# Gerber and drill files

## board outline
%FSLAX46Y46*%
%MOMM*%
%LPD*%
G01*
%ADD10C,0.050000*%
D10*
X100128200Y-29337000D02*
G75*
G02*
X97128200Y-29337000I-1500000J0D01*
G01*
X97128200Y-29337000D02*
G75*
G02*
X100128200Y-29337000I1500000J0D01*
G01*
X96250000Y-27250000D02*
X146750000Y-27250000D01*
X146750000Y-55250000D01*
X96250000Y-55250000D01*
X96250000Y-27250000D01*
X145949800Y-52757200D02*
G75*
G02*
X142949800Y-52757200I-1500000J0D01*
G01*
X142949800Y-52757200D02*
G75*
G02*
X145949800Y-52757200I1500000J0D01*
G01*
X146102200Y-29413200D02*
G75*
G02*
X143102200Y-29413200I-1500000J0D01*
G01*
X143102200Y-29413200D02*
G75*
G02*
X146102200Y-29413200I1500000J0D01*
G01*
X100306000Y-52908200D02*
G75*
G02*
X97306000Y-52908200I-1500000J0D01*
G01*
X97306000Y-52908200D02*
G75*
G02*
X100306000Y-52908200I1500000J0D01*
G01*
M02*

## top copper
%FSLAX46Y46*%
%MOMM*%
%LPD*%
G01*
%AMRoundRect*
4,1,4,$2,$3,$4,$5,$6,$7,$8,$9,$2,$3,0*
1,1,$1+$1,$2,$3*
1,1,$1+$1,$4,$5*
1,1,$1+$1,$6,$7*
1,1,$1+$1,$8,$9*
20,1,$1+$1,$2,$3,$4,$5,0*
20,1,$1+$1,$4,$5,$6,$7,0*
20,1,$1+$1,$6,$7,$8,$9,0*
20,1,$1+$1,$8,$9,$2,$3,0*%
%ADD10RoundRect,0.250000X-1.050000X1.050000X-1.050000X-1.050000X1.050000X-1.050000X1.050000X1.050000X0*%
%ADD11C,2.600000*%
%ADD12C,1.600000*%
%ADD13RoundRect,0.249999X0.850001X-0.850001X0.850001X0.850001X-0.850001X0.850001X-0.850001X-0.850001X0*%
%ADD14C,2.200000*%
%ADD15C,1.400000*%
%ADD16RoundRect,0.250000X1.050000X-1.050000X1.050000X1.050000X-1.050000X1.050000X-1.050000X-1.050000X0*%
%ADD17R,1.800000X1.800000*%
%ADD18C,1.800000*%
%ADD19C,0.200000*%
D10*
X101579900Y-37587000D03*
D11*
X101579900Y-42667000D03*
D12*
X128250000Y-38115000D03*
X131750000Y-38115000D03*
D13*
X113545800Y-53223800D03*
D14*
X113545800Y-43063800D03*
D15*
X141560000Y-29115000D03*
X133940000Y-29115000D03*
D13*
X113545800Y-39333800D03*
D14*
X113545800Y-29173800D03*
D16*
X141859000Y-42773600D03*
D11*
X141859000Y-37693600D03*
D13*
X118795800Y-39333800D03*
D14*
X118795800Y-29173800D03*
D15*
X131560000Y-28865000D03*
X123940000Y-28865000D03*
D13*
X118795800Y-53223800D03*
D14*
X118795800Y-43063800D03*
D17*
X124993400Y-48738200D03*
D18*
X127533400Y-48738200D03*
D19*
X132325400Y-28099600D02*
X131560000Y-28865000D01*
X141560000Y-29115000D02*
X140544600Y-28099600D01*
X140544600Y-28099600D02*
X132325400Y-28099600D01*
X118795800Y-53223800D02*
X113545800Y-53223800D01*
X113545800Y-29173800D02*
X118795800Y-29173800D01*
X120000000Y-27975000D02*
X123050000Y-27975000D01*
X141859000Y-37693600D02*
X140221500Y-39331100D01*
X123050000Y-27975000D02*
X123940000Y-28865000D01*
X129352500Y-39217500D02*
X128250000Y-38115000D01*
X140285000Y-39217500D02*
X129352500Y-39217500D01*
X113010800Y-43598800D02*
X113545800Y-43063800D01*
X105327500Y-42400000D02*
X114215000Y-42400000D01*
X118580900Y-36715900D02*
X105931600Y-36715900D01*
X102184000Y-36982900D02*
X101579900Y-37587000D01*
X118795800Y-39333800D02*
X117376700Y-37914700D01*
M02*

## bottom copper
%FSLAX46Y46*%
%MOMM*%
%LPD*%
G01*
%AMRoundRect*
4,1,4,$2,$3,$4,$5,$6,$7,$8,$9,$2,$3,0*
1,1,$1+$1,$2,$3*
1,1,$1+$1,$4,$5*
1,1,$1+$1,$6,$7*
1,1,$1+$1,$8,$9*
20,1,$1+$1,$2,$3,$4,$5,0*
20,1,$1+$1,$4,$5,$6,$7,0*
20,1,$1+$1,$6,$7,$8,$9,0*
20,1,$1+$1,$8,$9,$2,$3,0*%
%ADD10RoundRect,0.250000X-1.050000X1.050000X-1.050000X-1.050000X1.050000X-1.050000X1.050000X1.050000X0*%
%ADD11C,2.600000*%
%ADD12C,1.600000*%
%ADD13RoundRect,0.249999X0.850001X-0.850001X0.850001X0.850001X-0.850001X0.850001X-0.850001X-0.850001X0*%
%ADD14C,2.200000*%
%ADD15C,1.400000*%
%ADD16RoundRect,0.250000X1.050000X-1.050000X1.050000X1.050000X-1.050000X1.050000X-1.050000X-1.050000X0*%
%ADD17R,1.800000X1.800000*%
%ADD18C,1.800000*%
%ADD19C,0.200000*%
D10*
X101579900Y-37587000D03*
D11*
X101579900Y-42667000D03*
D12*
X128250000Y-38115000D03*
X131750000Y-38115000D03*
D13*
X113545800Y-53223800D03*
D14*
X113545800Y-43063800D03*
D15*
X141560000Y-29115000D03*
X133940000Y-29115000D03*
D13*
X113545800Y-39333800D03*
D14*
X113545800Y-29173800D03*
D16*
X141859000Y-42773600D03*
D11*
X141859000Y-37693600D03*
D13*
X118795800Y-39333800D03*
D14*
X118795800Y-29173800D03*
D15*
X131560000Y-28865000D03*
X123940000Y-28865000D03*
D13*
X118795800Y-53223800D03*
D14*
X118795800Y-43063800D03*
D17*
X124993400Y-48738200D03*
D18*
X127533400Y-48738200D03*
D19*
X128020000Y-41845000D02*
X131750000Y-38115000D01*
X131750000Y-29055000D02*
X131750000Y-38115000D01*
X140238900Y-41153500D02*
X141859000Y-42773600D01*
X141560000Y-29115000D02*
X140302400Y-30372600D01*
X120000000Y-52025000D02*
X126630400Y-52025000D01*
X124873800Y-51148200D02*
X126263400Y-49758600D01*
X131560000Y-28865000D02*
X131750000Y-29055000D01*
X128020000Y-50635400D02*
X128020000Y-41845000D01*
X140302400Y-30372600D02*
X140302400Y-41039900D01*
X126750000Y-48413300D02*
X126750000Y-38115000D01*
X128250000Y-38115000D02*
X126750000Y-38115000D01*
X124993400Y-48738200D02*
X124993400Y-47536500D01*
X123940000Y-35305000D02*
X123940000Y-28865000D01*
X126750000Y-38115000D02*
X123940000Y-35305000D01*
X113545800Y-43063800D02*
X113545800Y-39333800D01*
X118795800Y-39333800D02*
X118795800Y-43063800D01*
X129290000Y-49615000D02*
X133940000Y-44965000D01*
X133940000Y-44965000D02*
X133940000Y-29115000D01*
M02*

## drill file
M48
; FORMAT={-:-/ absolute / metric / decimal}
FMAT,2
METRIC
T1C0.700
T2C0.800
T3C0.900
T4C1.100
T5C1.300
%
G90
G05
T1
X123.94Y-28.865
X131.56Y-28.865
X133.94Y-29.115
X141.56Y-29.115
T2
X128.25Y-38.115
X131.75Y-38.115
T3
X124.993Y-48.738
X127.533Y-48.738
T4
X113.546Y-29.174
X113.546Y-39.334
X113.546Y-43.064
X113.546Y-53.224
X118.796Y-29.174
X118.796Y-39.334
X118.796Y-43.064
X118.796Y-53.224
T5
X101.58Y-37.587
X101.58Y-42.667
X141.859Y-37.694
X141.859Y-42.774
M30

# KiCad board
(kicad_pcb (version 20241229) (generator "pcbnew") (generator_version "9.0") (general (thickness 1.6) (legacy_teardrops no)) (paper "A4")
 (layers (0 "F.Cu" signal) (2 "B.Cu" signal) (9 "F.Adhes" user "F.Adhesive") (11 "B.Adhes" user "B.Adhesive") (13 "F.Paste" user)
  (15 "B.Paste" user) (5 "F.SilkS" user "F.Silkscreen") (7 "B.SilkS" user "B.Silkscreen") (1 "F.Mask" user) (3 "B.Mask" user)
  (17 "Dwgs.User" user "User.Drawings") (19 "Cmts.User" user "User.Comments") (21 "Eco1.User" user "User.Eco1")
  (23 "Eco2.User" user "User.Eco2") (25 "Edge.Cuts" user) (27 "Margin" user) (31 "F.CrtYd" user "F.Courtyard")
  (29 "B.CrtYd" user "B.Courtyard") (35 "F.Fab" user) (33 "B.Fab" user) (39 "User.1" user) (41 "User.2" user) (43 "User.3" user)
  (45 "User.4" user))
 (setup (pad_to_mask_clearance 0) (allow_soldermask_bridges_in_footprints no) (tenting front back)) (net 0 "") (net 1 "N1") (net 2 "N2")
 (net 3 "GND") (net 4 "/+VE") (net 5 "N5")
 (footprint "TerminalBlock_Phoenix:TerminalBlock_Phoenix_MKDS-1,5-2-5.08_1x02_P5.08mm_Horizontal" (layer "F.Cu") (at 101.5799 37.587 -90)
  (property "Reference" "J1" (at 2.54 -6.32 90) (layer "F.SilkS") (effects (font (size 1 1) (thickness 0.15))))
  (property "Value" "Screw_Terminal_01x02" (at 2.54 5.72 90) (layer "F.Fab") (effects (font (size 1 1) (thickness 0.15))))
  (pad "1" thru_hole roundrect (at 0 0 270) (size 2.6 2.6) (drill 1.3) (layers "*.Cu" "*.Mask") (remove_unused_layers no)
   (roundrect_rratio 0.096154) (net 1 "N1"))
  (pad "2" thru_hole circle (at 5.08 0 270) (size 2.6 2.6) (drill 1.3) (layers "*.Cu" "*.Mask") (remove_unused_layers no) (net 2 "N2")))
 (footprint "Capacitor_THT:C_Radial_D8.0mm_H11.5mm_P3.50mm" (layer "F.Cu") (at 128.25 38.115)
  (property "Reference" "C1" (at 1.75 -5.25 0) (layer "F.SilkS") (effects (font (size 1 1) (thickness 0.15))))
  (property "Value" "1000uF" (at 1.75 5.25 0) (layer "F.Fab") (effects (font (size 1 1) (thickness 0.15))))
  (pad "1" thru_hole circle (at 0 0) (size 1.6 1.6) (drill 0.8) (layers "*.Cu" "*.Mask") (remove_unused_layers no) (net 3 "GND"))
  (pad "2" thru_hole circle (at 3.5 0) (size 1.6 1.6) (drill 0.8) (layers "*.Cu" "*.Mask") (remove_unused_layers no) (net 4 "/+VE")))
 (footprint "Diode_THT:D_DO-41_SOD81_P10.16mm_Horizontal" (layer "F.Cu") (at 113.5458 53.2238 90)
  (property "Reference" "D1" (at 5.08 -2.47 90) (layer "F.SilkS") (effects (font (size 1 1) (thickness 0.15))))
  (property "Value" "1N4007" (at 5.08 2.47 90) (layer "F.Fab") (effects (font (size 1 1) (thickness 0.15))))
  (pad "1" thru_hole roundrect (at 0 0 90) (size 2.2 2.2) (drill 1.1) (layers "*.Cu" "*.Mask") (remove_unused_layers no)
   (roundrect_rratio 0.113636) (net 4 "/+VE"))
  (pad "2" thru_hole circle (at 10.16 0 90) (size 2.2 2.2) (drill 1.1) (layers "*.Cu" "*.Mask") (remove_unused_layers no) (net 2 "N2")))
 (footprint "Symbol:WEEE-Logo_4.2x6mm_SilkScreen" (layer "F.Cu") (at 102.4382 30.6578)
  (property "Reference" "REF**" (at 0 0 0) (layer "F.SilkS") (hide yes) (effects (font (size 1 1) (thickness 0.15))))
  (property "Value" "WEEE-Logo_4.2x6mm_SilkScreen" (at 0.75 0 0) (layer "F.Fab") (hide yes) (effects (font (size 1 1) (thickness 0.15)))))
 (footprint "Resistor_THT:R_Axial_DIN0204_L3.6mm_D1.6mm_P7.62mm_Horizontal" (layer "F.Cu") (at 141.56 29.115 180)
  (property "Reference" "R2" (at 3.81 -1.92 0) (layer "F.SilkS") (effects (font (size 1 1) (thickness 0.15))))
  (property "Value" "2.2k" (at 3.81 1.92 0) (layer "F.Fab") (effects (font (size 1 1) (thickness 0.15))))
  (pad "1" thru_hole circle (at 0 0 180) (size 1.4 1.4) (drill 0.7) (layers "*.Cu" "*.Mask") (remove_unused_layers no) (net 4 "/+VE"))
  (pad "2" thru_hole circle (at 7.62 0 180) (size 1.4 1.4) (drill 0.7) (layers "*.Cu" "*.Mask") (remove_unused_layers no) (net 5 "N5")))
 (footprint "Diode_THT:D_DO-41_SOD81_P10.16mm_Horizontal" (layer "F.Cu") (at 113.5458 39.3338 90)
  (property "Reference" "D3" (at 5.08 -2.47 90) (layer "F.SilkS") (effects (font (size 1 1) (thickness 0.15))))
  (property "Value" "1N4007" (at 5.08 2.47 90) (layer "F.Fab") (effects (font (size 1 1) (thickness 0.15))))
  (pad "1" thru_hole roundrect (at 0 0 90) (size 2.2 2.2) (drill 1.1) (layers "*.Cu" "*.Mask") (remove_unused_layers no)
   (roundrect_rratio 0.113636) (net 2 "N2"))
  (pad "2" thru_hole circle (at 10.16 0 90) (size 2.2 2.2) (drill 1.1) (layers "*.Cu" "*.Mask") (remove_unused_layers no) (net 3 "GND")))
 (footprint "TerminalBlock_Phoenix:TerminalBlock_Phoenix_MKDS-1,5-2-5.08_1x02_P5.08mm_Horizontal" (layer "F.Cu") (at 141.859 42.7736 90)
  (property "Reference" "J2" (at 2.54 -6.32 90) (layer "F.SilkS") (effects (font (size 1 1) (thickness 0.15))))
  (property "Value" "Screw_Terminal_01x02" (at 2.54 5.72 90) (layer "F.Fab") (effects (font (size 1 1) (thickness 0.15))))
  (pad "1" thru_hole roundrect (at 0 0 90) (size 2.6 2.6) (drill 1.3) (layers "*.Cu" "*.Mask") (remove_unused_layers no)
   (roundrect_rratio 0.096154) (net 4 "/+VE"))
  (pad "2" thru_hole circle (at 5.08 0 90) (size 2.6 2.6) (drill 1.3) (layers "*.Cu" "*.Mask") (remove_unused_layers no) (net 3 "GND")))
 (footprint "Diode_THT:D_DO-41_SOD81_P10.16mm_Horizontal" (layer "F.Cu") (at 118.7958 39.3338 90)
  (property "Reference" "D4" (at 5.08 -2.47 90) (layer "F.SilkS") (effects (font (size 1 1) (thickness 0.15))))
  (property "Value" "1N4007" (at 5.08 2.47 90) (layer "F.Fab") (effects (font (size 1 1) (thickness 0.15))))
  (pad "1" thru_hole roundrect (at 0 0 90) (size 2.2 2.2) (drill 1.1) (layers "*.Cu" "*.Mask") (remove_unused_layers no)
   (roundrect_rratio 0.113636) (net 1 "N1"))
  (pad "2" thru_hole circle (at 10.16 0 90) (size 2.2 2.2) (drill 1.1) (layers "*.Cu" "*.Mask") (remove_unused_layers no) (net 3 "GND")))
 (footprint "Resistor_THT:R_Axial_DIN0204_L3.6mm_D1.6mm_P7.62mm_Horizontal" (layer "F.Cu") (at 131.56 28.865 180)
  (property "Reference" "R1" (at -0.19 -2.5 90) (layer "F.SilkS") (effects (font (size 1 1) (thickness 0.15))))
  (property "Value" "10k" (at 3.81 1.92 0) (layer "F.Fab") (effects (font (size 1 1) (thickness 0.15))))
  (pad "1" thru_hole circle (at 0 0 180) (size 1.4 1.4) (drill 0.7) (layers "*.Cu" "*.Mask") (remove_unused_layers no) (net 4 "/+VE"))
  (pad "2" thru_hole circle (at 7.62 0 180) (size 1.4 1.4) (drill 0.7) (layers "*.Cu" "*.Mask") (remove_unused_layers no) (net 3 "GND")))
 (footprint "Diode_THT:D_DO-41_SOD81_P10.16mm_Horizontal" (layer "F.Cu") (at 118.7958 53.2238 90)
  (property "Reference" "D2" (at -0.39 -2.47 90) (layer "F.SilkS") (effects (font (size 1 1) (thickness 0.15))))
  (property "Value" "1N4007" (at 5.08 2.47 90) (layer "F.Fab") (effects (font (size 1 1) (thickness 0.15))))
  (pad "1" thru_hole roundrect (at 0 0 90) (size 2.2 2.2) (drill 1.1) (layers "*.Cu" "*.Mask") (remove_unused_layers no)
   (roundrect_rratio 0.113636) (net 4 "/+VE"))
  (pad "2" thru_hole circle (at 10.16 0 90) (size 2.2 2.2) (drill 1.1) (layers "*.Cu" "*.Mask") (remove_unused_layers no) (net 1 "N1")))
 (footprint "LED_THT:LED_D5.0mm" (layer "F.Cu") (at 124.9934 48.7382)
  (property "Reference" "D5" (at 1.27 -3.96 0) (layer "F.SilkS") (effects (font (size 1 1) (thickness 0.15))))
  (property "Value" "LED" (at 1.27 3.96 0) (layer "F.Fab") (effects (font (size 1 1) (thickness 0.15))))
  (pad "1" thru_hole rect (at 0 0) (size 1.8 1.8) (drill 0.9) (layers "*.Cu" "*.Mask") (remove_unused_layers no) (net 3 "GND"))
  (pad "2" thru_hole circle (at 2.54 0) (size 1.8 1.8) (drill 0.9) (layers "*.Cu" "*.Mask") (remove_unused_layers no) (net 5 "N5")))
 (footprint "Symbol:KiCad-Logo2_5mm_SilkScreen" (layer "B.Cu") (at 121.5 41.25 180)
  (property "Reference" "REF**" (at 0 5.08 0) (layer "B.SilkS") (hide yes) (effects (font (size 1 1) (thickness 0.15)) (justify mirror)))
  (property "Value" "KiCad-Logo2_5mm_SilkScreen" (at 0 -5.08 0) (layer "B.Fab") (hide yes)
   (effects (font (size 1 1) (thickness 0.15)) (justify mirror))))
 (gr_circle (center 98.6282 29.337) (end 100.1282 29.337) (stroke (width 0.05) (type solid)) (fill no) (layer "Edge.Cuts"))
 (gr_rect (start 96.25 27.25) (end 146.75 55.25) (stroke (width 0.05) (type default)) (fill no) (locked yes) (layer "Edge.Cuts"))
 (gr_circle (center 144.4498 52.7572) (end 145.9498 52.7572) (stroke (width 0.05) (type solid)) (fill no) (layer "Edge.Cuts"))
 (gr_circle (center 144.6022 29.4132) (end 146.1022 29.4132) (stroke (width 0.05) (type solid)) (fill no) (layer "Edge.Cuts"))
 (gr_circle (center 98.806 52.9082) (end 100.306 52.9082) (stroke (width 0.05) (type solid)) (fill no) (layer "Edge.Cuts"))
 (segment (start 132.3254 28.0996) (end 131.56 28.865) (width 0.2) (layer "F.Cu") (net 4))
 (segment (start 141.56 29.115) (end 140.5446 28.0996) (width 0.2) (layer "F.Cu") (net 4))
 (segment (start 140.5446 28.0996) (end 132.3254 28.0996) (width 0.2) (layer "F.Cu") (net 4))
 (segment (start 118.7958 53.2238) (end 113.5458 53.2238) (width 0.2) (layer "F.Cu") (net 4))
 (segment (start 128.02 41.845) (end 131.75 38.115) (width 0.2) (layer "B.Cu") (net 4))
 (segment (start 131.75 29.055) (end 131.75 38.115) (width 0.2) (layer "B.Cu") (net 4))
 (segment (start 140.2389 41.1535) (end 141.859 42.7736) (width 0.2) (layer "B.Cu") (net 4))
 (segment (start 141.56 29.115) (end 140.3024 30.3726) (width 0.2) (layer "B.Cu") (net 4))
 (segment (start 120 52.025) (end 126.6304 52.025) (width 0.2) (layer "B.Cu") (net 4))
 (segment (start 124.8738 51.1482) (end 126.2634 49.7586) (width 0.2) (layer "B.Cu") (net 4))
 (segment (start 131.56 28.865) (end 131.75 29.055) (width 0.2) (layer "B.Cu") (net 4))
 (segment (start 128.02 50.6354) (end 128.02 41.845) (width 0.2) (layer "B.Cu") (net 4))
 (segment (start 140.3024 30.3726) (end 140.3024 41.0399) (width 0.2) (layer "B.Cu") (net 4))
 (segment (start 113.5458 29.1738) (end 118.7958 29.1738) (width 0.2) (layer "F.Cu") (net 3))
 (segment (start 120 27.975) (end 123.05 27.975) (width 0.2) (layer "F.Cu") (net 3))
 (segment (start 141.859 37.6936) (end 140.2215 39.3311) (width 0.2) (layer "F.Cu") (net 3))
 (segment (start 123.05 27.975) (end 123.94 28.865) (width 0.2) (layer "F.Cu") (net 3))
 (segment (start 129.3525 39.2175) (end 128.25 38.115) (width 0.2) (layer "F.Cu") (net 3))
 (segment (start 140.285 39.2175) (end 129.3525 39.2175) (width 0.2) (layer "F.Cu") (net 3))
 (segment (start 126.75 48.4133) (end 126.75 38.115) (width 0.2) (layer "B.Cu") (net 3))
 (segment (start 128.25 38.115) (end 126.75 38.115) (width 0.2) (layer "B.Cu") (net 3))
 (segment (start 124.9934 48.7382) (end 124.9934 47.5365) (width 0.2) (layer "B.Cu") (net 3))
 (segment (start 123.94 35.305) (end 123.94 28.865) (width 0.2) (layer "B.Cu") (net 3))
 (segment (start 126.75 38.115) (end 123.94 35.305) (width 0.2) (layer "B.Cu") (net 3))
 (segment (start 113.0108 43.5988) (end 113.5458 43.0638) (width 0.2) (layer "F.Cu") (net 2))
 (segment (start 105.3275 42.4) (end 114.215 42.4) (width 0.2) (layer "F.Cu") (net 2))
 (segment (start 113.5458 43.0638) (end 113.5458 39.3338) (width 0.2) (layer "B.Cu") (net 2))
 (segment (start 118.5809 36.7159) (end 105.9316 36.7159) (width 0.2) (layer "F.Cu") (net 1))
 (segment (start 102.184 36.9829) (end 101.5799 37.587) (width 0.2) (layer "F.Cu") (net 1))
 (segment (start 118.7958 39.3338) (end 117.3767 37.9147) (width 0.2) (layer "F.Cu") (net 1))
 (segment (start 118.7958 39.3338) (end 118.7958 43.0638) (width 0.2) (layer "B.Cu") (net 1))
 (segment (start 129.29 49.615) (end 133.94 44.965) (width 0.2) (layer "B.Cu") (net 5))
 (segment (start 133.94 44.965) (end 133.94 29.115) (width 0.2) (layer "B.Cu") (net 5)))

